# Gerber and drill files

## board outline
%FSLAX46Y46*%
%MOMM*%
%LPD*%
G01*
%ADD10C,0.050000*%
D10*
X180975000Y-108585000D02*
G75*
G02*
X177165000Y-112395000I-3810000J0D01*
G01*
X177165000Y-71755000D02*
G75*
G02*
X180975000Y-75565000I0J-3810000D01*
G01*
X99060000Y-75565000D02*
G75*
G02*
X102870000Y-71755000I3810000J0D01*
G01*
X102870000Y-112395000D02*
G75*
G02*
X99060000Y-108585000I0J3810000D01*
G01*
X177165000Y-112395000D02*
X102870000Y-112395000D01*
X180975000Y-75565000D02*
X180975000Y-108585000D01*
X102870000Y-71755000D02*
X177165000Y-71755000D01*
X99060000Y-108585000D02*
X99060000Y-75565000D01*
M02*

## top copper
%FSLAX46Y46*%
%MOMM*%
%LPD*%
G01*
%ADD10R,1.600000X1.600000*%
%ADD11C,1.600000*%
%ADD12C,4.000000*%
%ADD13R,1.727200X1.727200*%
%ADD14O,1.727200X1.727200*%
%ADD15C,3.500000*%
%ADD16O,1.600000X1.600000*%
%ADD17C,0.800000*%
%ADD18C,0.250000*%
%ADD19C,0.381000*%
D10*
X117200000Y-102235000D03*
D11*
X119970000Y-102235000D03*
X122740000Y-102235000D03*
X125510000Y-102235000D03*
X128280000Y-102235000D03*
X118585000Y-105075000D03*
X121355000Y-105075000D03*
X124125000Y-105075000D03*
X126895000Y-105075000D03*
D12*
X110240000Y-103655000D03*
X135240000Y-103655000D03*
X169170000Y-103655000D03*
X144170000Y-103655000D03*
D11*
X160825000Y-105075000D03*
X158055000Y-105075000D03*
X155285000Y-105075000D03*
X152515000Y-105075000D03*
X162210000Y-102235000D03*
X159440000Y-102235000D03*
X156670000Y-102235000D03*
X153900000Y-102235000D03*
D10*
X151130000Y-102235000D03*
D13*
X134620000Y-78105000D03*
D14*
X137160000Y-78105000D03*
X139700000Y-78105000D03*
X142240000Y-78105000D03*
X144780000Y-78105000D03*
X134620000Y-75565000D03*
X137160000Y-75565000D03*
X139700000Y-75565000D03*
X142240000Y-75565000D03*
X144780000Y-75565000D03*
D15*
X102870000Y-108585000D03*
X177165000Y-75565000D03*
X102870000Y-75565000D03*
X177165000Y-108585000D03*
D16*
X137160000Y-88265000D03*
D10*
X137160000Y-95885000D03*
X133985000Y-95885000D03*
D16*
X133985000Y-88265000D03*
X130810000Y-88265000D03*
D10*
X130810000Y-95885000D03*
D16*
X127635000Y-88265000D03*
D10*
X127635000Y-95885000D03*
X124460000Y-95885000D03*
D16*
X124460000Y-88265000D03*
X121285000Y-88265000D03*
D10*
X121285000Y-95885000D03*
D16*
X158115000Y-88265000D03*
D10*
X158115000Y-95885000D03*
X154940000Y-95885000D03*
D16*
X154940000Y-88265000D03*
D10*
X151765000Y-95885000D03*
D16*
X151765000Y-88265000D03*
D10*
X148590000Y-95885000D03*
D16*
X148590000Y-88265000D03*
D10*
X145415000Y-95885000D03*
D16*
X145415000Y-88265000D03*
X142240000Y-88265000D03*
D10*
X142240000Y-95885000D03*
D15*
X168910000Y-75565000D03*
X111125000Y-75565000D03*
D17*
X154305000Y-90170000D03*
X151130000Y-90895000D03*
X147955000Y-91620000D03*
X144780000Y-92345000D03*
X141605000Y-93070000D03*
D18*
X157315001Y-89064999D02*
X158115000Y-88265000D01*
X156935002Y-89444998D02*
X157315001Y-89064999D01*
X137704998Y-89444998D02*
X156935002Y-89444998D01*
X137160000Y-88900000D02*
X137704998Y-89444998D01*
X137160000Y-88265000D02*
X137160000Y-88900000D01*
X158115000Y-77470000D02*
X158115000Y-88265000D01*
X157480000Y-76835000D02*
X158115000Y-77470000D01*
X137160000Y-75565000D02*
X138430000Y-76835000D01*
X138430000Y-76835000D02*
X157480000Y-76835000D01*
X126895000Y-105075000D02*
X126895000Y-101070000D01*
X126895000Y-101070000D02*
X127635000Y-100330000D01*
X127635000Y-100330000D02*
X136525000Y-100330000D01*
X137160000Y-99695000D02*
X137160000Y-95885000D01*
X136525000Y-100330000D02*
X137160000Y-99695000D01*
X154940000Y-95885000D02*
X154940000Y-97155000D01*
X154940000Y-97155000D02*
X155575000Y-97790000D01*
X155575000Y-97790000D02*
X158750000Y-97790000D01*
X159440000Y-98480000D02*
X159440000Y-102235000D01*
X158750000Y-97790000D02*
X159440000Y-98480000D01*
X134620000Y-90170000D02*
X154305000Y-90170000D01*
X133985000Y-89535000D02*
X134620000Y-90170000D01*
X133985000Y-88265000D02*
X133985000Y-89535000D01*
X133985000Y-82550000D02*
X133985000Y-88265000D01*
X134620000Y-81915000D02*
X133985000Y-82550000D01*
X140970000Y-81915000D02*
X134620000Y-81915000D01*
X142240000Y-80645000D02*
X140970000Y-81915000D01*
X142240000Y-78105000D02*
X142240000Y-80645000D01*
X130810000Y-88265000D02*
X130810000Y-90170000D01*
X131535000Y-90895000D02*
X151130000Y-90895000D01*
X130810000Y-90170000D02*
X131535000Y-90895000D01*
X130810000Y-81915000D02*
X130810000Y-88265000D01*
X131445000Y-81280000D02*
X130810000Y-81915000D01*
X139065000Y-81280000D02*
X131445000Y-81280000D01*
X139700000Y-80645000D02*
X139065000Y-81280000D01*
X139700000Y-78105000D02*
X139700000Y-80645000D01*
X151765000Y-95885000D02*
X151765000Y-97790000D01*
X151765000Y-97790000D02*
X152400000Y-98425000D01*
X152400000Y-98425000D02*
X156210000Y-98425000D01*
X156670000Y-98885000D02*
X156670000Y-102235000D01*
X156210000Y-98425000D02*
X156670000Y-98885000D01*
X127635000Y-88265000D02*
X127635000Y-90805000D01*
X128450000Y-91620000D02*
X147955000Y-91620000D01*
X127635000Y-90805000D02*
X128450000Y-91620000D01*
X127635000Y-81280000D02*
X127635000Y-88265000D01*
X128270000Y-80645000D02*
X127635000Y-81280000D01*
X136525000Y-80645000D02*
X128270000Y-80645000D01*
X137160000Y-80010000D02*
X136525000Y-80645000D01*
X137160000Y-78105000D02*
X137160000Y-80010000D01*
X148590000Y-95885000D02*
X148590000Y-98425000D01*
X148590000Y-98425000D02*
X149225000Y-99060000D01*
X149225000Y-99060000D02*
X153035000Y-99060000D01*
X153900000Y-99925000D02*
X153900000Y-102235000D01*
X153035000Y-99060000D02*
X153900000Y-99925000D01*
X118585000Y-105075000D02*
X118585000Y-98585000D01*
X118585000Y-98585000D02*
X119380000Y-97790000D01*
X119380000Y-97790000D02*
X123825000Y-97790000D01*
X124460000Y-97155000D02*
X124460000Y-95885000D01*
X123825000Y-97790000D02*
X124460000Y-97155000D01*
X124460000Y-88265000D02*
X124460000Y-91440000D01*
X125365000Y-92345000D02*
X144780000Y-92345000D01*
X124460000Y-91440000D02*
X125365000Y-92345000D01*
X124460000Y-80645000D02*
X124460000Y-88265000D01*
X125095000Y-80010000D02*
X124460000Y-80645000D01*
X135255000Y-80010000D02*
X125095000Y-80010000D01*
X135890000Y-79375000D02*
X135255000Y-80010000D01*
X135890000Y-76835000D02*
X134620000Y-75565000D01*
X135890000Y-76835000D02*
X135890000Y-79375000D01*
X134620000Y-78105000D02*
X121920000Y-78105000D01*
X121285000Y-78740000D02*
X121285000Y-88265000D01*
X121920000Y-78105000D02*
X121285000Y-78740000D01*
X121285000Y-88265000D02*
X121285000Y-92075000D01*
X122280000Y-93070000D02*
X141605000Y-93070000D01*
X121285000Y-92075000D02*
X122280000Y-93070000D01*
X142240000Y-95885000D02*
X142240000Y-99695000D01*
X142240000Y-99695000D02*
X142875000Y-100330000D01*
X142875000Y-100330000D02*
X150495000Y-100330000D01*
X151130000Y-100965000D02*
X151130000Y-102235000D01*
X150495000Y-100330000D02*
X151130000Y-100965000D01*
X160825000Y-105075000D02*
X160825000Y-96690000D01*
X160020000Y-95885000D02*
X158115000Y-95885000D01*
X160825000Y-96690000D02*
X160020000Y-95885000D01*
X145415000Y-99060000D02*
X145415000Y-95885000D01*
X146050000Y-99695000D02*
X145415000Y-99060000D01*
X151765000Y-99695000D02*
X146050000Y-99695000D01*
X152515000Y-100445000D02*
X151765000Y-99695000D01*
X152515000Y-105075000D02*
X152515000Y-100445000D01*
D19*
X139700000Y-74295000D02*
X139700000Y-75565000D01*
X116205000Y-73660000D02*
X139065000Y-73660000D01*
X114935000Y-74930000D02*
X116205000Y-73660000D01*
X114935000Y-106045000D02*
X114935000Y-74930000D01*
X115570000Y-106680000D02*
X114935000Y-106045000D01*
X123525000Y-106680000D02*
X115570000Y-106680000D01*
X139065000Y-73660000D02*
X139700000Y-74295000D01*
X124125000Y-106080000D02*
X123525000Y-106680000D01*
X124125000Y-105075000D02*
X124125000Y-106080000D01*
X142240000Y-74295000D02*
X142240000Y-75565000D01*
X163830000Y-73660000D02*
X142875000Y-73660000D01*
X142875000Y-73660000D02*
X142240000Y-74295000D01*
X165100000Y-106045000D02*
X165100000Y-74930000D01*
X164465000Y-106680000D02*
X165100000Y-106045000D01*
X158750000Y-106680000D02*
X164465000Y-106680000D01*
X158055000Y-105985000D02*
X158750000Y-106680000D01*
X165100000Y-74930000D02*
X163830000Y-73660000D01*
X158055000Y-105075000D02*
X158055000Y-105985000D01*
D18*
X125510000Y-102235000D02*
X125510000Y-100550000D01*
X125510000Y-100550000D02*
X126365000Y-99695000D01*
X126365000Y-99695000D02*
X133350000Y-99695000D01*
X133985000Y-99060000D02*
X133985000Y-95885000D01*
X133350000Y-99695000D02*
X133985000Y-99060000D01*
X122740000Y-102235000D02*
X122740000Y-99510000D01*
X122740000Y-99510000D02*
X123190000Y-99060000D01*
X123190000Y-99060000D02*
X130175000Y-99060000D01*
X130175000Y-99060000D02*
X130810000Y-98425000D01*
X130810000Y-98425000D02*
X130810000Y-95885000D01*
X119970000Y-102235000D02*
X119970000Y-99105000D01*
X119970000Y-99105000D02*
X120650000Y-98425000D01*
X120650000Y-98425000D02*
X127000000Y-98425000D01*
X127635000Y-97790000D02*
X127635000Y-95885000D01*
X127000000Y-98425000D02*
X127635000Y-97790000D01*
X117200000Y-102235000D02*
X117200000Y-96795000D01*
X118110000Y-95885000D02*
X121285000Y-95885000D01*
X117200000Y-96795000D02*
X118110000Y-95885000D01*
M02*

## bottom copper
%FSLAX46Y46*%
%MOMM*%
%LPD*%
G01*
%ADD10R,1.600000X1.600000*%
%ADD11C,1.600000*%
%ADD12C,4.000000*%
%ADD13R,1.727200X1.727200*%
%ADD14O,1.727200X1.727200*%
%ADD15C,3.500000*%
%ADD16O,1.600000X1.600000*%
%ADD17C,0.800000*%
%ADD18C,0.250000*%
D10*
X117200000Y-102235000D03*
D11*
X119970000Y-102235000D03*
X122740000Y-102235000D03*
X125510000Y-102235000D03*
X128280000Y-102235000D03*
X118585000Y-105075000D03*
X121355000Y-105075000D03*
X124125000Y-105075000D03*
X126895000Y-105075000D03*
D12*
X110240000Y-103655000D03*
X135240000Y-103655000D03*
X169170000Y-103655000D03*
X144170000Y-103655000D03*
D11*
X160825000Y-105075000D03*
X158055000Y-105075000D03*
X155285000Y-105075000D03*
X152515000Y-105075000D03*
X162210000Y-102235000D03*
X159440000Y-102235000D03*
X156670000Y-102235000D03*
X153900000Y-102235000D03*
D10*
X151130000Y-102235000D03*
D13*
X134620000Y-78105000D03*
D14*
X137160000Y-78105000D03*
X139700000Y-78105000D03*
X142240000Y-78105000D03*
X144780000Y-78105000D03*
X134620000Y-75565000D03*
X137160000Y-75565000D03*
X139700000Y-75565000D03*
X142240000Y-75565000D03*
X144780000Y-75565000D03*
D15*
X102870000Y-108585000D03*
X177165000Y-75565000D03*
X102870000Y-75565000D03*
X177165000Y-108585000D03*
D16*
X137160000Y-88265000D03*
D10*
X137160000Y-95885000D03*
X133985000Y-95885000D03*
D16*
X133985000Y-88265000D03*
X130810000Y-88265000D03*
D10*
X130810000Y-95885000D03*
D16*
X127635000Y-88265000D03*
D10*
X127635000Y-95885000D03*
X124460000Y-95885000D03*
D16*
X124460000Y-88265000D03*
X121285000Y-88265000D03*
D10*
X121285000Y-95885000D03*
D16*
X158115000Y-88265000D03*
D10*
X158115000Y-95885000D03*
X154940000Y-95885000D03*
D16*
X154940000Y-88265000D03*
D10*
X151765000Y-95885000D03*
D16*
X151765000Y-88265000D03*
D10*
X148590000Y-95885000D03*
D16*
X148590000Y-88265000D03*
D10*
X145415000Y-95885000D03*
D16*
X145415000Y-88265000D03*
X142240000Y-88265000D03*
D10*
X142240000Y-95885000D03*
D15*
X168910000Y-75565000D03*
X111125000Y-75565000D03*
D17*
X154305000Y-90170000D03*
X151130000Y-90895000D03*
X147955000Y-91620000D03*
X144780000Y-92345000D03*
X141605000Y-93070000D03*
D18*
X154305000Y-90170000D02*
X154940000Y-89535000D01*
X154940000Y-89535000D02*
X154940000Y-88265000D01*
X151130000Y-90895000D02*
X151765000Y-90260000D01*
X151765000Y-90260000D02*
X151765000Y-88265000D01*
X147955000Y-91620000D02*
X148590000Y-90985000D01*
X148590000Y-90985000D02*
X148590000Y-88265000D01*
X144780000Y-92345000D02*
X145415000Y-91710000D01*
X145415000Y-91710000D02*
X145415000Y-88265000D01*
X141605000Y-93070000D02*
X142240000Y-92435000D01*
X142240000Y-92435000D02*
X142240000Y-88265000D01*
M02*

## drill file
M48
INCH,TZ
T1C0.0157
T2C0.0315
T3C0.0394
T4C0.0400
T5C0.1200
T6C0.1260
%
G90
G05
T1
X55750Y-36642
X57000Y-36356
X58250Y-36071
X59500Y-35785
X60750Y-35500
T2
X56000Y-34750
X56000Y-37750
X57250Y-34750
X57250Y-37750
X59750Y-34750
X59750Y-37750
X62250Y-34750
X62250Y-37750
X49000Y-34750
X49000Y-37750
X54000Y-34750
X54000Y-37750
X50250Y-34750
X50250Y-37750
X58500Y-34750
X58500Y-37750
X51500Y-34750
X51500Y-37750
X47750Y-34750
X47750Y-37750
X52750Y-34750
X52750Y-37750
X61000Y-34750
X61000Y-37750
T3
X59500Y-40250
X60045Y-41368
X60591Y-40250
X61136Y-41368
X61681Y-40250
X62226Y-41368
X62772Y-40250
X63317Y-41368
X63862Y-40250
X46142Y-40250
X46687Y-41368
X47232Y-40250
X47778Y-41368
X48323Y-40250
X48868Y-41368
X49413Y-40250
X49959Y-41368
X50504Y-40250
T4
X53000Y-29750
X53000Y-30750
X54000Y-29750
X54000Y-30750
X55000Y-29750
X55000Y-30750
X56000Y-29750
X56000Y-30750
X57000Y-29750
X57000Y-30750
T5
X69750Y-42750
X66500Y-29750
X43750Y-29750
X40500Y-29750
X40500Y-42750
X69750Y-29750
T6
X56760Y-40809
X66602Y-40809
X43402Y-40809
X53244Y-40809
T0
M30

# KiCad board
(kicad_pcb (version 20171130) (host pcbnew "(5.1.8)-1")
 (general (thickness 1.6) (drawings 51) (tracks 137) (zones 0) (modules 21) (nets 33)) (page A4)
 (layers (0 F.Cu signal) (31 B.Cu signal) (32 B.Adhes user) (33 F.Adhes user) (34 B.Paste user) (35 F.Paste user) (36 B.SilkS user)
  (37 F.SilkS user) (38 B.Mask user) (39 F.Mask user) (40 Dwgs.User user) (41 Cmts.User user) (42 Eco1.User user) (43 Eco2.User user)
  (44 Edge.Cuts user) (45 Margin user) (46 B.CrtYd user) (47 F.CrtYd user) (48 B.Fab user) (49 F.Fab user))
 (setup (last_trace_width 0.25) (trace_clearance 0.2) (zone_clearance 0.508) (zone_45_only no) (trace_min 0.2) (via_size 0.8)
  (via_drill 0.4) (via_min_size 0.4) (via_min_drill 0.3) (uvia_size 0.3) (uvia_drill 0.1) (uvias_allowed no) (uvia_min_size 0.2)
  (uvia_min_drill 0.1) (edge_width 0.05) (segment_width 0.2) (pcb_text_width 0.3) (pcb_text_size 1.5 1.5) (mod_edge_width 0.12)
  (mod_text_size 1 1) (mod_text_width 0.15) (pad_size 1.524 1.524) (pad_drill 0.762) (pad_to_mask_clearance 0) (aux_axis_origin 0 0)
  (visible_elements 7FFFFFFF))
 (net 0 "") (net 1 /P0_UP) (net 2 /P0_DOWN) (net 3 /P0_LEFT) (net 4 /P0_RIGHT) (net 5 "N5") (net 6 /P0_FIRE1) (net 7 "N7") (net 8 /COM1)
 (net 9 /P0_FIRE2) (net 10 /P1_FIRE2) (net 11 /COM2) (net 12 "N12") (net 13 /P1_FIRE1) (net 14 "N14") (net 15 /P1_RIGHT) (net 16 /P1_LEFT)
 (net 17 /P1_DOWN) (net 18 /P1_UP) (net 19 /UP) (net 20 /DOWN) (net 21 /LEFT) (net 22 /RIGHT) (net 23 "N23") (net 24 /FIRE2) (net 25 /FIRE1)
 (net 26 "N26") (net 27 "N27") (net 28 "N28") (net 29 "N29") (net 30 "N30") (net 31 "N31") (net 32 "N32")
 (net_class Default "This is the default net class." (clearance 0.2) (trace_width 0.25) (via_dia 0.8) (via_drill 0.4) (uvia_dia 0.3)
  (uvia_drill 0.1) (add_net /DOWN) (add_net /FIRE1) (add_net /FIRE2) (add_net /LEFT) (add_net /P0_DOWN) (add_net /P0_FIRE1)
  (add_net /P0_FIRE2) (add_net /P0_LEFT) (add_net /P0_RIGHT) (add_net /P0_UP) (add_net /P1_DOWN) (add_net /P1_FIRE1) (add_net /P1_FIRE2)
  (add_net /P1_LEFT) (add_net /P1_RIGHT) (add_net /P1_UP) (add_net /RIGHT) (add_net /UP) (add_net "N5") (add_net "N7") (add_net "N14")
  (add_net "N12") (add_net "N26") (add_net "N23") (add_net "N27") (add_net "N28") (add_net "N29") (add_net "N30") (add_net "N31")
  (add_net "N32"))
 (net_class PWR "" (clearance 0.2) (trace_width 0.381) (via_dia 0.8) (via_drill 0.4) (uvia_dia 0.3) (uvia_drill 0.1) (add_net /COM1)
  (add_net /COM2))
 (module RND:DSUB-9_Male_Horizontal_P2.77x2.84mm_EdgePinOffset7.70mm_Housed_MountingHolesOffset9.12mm (layer F.Cu) (at 117.2 102.235)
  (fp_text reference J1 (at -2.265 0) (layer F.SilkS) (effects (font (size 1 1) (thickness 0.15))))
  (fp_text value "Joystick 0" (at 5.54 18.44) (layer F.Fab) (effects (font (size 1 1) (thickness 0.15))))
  (pad 1 thru_hole rect (at 0 0) (size 1.6 1.6) (drill 1) (layers *.Cu *.Mask) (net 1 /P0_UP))
  (pad 2 thru_hole circle (at 2.77 0) (size 1.6 1.6) (drill 1) (layers *.Cu *.Mask) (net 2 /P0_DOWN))
  (pad 3 thru_hole circle (at 5.54 0) (size 1.6 1.6) (drill 1) (layers *.Cu *.Mask) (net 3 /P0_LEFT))
  (pad 4 thru_hole circle (at 8.31 0) (size 1.6 1.6) (drill 1) (layers *.Cu *.Mask) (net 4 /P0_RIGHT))
  (pad 5 thru_hole circle (at 11.08 0) (size 1.6 1.6) (drill 1) (layers *.Cu *.Mask) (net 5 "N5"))
  (pad 6 thru_hole circle (at 1.385 2.84) (size 1.6 1.6) (drill 1) (layers *.Cu *.Mask) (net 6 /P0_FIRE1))
  (pad 7 thru_hole circle (at 4.155 2.84) (size 1.6 1.6) (drill 1) (layers *.Cu *.Mask) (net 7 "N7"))
  (pad 8 thru_hole circle (at 6.925 2.84) (size 1.6 1.6) (drill 1) (layers *.Cu *.Mask) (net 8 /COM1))
  (pad 9 thru_hole circle (at 9.695 2.84) (size 1.6 1.6) (drill 1) (layers *.Cu *.Mask) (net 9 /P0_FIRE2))
  (pad 0 thru_hole circle (at -6.96 1.42) (size 4 4) (drill 3.2) (layers *.Cu *.Mask))
  (pad 0 thru_hole circle (at 18.04 1.42) (size 4 4) (drill 3.2) (layers *.Cu *.Mask)))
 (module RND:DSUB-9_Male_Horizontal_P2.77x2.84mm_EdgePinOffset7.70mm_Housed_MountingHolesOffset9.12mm (layer F.Cu) (at 151.13 102.235)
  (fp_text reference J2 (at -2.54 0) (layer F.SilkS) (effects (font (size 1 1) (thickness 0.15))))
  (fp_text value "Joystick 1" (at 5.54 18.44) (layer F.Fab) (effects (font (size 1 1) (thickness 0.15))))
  (pad 0 thru_hole circle (at 18.04 1.42) (size 4 4) (drill 3.2) (layers *.Cu *.Mask))
  (pad 0 thru_hole circle (at -6.96 1.42) (size 4 4) (drill 3.2) (layers *.Cu *.Mask))
  (pad 9 thru_hole circle (at 9.695 2.84) (size 1.6 1.6) (drill 1) (layers *.Cu *.Mask) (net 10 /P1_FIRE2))
  (pad 8 thru_hole circle (at 6.925 2.84) (size 1.6 1.6) (drill 1) (layers *.Cu *.Mask) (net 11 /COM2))
  (pad 7 thru_hole circle (at 4.155 2.84) (size 1.6 1.6) (drill 1) (layers *.Cu *.Mask) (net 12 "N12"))
  (pad 6 thru_hole circle (at 1.385 2.84) (size 1.6 1.6) (drill 1) (layers *.Cu *.Mask) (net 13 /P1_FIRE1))
  (pad 5 thru_hole circle (at 11.08 0) (size 1.6 1.6) (drill 1) (layers *.Cu *.Mask) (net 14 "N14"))
  (pad 4 thru_hole circle (at 8.31 0) (size 1.6 1.6) (drill 1) (layers *.Cu *.Mask) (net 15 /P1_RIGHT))
  (pad 3 thru_hole circle (at 5.54 0) (size 1.6 1.6) (drill 1) (layers *.Cu *.Mask) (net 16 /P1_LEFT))
  (pad 2 thru_hole circle (at 2.77 0) (size 1.6 1.6) (drill 1) (layers *.Cu *.Mask) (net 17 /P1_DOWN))
  (pad 1 thru_hole rect (at 0 0) (size 1.6 1.6) (drill 1) (layers *.Cu *.Mask) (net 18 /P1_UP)))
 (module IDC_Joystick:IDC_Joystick (layer F.Cu) (at 134.62 78.105 90)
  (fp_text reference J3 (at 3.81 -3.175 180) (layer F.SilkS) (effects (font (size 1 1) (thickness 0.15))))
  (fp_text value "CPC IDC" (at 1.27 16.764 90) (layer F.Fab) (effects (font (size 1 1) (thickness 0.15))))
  (pad 1 thru_hole rect (at 0 0 90) (size 1.7272 1.7272) (drill 1.016) (layers *.Cu *.Mask) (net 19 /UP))
  (pad 2 thru_hole oval (at 0 2.54 90) (size 1.7272 1.7272) (drill 1.016) (layers *.Cu *.Mask) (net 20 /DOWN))
  (pad 3 thru_hole oval (at 0 5.08 90) (size 1.7272 1.7272) (drill 1.016) (layers *.Cu *.Mask) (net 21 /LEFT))
  (pad 4 thru_hole oval (at 0 7.62 90) (size 1.7272 1.7272) (drill 1.016) (layers *.Cu *.Mask) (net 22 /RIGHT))
  (pad 5 thru_hole oval (at 0 10.16 90) (size 1.7272 1.7272) (drill 1.016) (layers *.Cu *.Mask) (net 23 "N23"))
  (pad 6 thru_hole oval (at 2.54 0 90) (size 1.7272 1.7272) (drill 1.016) (layers *.Cu *.Mask) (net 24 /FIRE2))
  (pad 7 thru_hole oval (at 2.54 2.54 90) (size 1.7272 1.7272) (drill 1.016) (layers *.Cu *.Mask) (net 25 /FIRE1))
  (pad 8 thru_hole oval (at 2.54 5.08 90) (size 1.7272 1.7272) (drill 1.016) (layers *.Cu *.Mask) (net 8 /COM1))
  (pad 9 thru_hole oval (at 2.54 7.62 90) (size 1.7272 1.7272) (drill 1.016) (layers *.Cu *.Mask) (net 11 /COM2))
  (pad 10 thru_hole oval (at 2.54 10.16 90) (size 1.7272 1.7272) (drill 1.016) (layers *.Cu *.Mask) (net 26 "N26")))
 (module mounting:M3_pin (layer F.Cu) (at 102.87 108.585)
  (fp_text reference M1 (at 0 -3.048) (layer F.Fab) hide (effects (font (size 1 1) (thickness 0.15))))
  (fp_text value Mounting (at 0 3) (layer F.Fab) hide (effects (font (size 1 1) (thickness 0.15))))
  (pad 1 thru_hole circle (at 0 0) (size 3.5 3.5) (drill 3.048) (layers *.Cu *.Mask) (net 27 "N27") (solder_mask_margin 0.8)))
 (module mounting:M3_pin (layer F.Cu) (at 177.165 75.565)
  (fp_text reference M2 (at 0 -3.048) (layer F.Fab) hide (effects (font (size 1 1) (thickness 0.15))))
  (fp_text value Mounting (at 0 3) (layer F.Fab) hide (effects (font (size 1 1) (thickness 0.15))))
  (pad 1 thru_hole circle (at 0 0) (size 3.5 3.5) (drill 3.048) (layers *.Cu *.Mask) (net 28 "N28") (solder_mask_margin 0.8)))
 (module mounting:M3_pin (layer F.Cu) (at 102.87 75.565)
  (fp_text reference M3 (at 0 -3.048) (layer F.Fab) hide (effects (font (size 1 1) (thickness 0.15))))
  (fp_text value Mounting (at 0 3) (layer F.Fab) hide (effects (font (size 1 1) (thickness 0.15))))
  (pad 1 thru_hole circle (at 0 0) (size 3.5 3.5) (drill 3.048) (layers *.Cu *.Mask) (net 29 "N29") (solder_mask_margin 0.8)))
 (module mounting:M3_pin (layer F.Cu) (at 177.165 108.585)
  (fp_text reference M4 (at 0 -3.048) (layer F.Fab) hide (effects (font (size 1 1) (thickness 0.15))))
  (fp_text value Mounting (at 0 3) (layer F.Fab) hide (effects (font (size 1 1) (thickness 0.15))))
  (pad 1 thru_hole circle (at 0 0) (size 3.5 3.5) (drill 3.048) (layers *.Cu *.Mask) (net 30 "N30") (solder_mask_margin 0.8)))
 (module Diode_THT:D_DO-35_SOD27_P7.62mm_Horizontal (layer F.Cu) (at 137.16 95.885 90)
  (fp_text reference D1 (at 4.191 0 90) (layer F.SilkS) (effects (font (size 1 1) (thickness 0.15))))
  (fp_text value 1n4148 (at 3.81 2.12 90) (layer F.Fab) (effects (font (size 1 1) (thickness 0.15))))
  (pad 2 thru_hole oval (at 7.62 0 90) (size 1.6 1.6) (drill 0.8) (layers *.Cu *.Mask) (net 25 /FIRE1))
  (pad 1 thru_hole rect (at 0 0 90) (size 1.6 1.6) (drill 0.8) (layers *.Cu *.Mask) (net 9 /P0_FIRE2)))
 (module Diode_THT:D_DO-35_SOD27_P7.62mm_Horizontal (layer F.Cu) (at 133.985 95.885 90)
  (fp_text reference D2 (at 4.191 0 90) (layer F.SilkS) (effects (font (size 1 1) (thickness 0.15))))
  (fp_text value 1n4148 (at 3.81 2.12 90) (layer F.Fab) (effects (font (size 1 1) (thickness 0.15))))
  (pad 1 thru_hole rect (at 0 0 90) (size 1.6 1.6) (drill 0.8) (layers *.Cu *.Mask) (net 4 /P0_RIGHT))
  (pad 2 thru_hole oval (at 7.62 0 90) (size 1.6 1.6) (drill 0.8) (layers *.Cu *.Mask) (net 22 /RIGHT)))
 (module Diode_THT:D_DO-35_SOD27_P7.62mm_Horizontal (layer F.Cu) (at 130.81 95.885 90)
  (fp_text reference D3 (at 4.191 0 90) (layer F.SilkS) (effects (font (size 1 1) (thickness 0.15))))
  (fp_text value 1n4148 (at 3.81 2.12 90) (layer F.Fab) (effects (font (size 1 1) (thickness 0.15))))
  (pad 2 thru_hole oval (at 7.62 0 90) (size 1.6 1.6) (drill 0.8) (layers *.Cu *.Mask) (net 21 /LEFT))
  (pad 1 thru_hole rect (at 0 0 90) (size 1.6 1.6) (drill 0.8) (layers *.Cu *.Mask) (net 3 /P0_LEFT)))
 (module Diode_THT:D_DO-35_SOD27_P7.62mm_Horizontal (layer F.Cu) (at 127.635 95.885 90)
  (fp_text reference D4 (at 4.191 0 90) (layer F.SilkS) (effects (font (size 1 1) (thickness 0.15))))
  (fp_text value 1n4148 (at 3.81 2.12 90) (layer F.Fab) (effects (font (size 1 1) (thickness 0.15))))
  (pad 2 thru_hole oval (at 7.62 0 90) (size 1.6 1.6) (drill 0.8) (layers *.Cu *.Mask) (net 20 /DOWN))
  (pad 1 thru_hole rect (at 0 0 90) (size 1.6 1.6) (drill 0.8) (layers *.Cu *.Mask) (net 2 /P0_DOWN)))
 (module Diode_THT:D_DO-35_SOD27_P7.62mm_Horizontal (layer F.Cu) (at 124.46 95.885 90)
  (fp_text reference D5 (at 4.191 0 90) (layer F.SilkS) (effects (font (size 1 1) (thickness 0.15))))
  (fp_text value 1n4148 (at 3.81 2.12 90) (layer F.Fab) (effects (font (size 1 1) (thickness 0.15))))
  (pad 1 thru_hole rect (at 0 0 90) (size 1.6 1.6) (drill 0.8) (layers *.Cu *.Mask) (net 6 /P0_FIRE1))
  (pad 2 thru_hole oval (at 7.62 0 90) (size 1.6 1.6) (drill 0.8) (layers *.Cu *.Mask) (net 24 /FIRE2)))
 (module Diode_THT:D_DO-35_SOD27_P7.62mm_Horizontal (layer F.Cu) (at 121.285 95.885 90)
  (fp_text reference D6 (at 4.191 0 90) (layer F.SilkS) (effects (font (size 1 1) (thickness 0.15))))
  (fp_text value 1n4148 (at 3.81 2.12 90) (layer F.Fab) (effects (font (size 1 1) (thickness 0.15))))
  (pad 2 thru_hole oval (at 7.62 0 90) (size 1.6 1.6) (drill 0.8) (layers *.Cu *.Mask) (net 19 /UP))
  (pad 1 thru_hole rect (at 0 0 90) (size 1.6 1.6) (drill 0.8) (layers *.Cu *.Mask) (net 1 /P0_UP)))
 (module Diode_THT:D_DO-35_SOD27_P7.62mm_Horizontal (layer F.Cu) (at 158.115 95.885 90)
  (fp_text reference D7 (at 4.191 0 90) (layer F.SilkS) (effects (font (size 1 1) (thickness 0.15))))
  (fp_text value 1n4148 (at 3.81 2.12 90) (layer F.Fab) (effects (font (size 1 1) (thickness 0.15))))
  (pad 2 thru_hole oval (at 7.62 0 90) (size 1.6 1.6) (drill 0.8) (layers *.Cu *.Mask) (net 25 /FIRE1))
  (pad 1 thru_hole rect (at 0 0 90) (size 1.6 1.6) (drill 0.8) (layers *.Cu *.Mask) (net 10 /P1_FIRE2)))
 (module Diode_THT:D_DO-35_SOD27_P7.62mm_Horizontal (layer F.Cu) (at 154.94 95.885 90)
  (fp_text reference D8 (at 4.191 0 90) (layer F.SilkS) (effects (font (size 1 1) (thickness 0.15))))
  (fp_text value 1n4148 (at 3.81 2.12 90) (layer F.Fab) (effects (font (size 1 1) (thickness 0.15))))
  (pad 1 thru_hole rect (at 0 0 90) (size 1.6 1.6) (drill 0.8) (layers *.Cu *.Mask) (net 15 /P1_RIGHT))
  (pad 2 thru_hole oval (at 7.62 0 90) (size 1.6 1.6) (drill 0.8) (layers *.Cu *.Mask) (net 22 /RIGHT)))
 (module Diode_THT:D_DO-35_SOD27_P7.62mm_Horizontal (layer F.Cu) (at 151.765 95.885 90)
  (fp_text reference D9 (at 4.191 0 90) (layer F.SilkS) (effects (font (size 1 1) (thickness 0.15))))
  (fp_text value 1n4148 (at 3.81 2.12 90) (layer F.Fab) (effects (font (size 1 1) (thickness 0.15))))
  (pad 1 thru_hole rect (at 0 0 90) (size 1.6 1.6) (drill 0.8) (layers *.Cu *.Mask) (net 16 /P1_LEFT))
  (pad 2 thru_hole oval (at 7.62 0 90) (size 1.6 1.6) (drill 0.8) (layers *.Cu *.Mask) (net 21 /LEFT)))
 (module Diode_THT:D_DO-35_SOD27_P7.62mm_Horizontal (layer F.Cu) (at 148.59 95.885 90)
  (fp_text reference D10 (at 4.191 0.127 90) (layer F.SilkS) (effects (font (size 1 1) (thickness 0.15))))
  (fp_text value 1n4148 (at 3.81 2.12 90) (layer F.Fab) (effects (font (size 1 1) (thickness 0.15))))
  (pad 1 thru_hole rect (at 0 0 90) (size 1.6 1.6) (drill 0.8) (layers *.Cu *.Mask) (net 17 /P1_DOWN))
  (pad 2 thru_hole oval (at 7.62 0 90) (size 1.6 1.6) (drill 0.8) (layers *.Cu *.Mask) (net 20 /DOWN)))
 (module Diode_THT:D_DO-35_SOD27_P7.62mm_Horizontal (layer F.Cu) (at 145.415 95.885 90)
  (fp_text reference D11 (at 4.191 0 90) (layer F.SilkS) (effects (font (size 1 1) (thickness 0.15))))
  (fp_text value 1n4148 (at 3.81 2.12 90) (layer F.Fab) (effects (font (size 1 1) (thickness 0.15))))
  (pad 1 thru_hole rect (at 0 0 90) (size 1.6 1.6) (drill 0.8) (layers *.Cu *.Mask) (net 13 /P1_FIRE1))
  (pad 2 thru_hole oval (at 7.62 0 90) (size 1.6 1.6) (drill 0.8) (layers *.Cu *.Mask) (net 24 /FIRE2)))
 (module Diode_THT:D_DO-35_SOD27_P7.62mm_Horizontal (layer F.Cu) (at 142.24 95.885 90)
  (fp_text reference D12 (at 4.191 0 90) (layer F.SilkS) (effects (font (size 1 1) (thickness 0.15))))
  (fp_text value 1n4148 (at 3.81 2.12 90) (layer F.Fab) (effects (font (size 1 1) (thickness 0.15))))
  (pad 2 thru_hole oval (at 7.62 0 90) (size 1.6 1.6) (drill 0.8) (layers *.Cu *.Mask) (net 19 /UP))
  (pad 1 thru_hole rect (at 0 0 90) (size 1.6 1.6) (drill 0.8) (layers *.Cu *.Mask) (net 18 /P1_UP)))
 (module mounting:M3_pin (layer F.Cu) (at 168.91 75.565)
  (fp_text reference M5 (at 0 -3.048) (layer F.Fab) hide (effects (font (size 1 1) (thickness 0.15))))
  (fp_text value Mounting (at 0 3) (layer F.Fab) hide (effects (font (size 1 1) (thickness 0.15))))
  (pad 1 thru_hole circle (at 0 0) (size 3.5 3.5) (drill 3.048) (layers *.Cu *.Mask) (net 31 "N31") (solder_mask_margin 0.8)))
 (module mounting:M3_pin (layer F.Cu) (at 111.125 75.565)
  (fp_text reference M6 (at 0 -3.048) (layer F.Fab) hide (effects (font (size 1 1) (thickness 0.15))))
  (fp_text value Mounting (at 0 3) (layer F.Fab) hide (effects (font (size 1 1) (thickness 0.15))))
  (pad 1 thru_hole circle (at 0 0) (size 3.5 3.5) (drill 3.048) (layers *.Cu *.Mask) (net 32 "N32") (solder_mask_margin 0.8)))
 (gr_arc (start 177.165 108.585) (end 177.165 112.395) (angle -90) (layer Edge.Cuts) (width 0.05))
 (gr_arc (start 177.165 75.565) (end 180.975 75.565) (angle -90) (layer Edge.Cuts) (width 0.05))
 (gr_arc (start 102.87 75.565) (end 102.87 71.755) (angle -90) (layer Edge.Cuts) (width 0.05))
 (gr_arc (start 102.87 108.585) (end 99.06 108.585) (angle -90) (layer Edge.Cuts) (width 0.05))
 (gr_line (start 177.165 112.395) (end 102.87 112.395) (layer Edge.Cuts) (width 0.05))
 (gr_line (start 180.975 75.565) (end 180.975 108.585) (layer Edge.Cuts) (width 0.05))
 (gr_line (start 102.87 71.755) (end 177.165 71.755) (layer Edge.Cuts) (width 0.05))
 (gr_line (start 99.06 108.585) (end 99.06 75.565) (layer Edge.Cuts) (width 0.05))
 (segment (start 157.315001 89.064999) (end 158.115 88.265) (width 0.25) (layer F.Cu) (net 25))
 (segment (start 156.935002 89.444998) (end 157.315001 89.064999) (width 0.25) (layer F.Cu) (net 25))
 (segment (start 137.704998 89.444998) (end 156.935002 89.444998) (width 0.25) (layer F.Cu) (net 25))
 (segment (start 137.16 88.9) (end 137.704998 89.444998) (width 0.25) (layer F.Cu) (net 25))
 (segment (start 137.16 88.265) (end 137.16 88.9) (width 0.25) (layer F.Cu) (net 25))
 (segment (start 158.115 77.47) (end 158.115 88.265) (width 0.25) (layer F.Cu) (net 25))
 (segment (start 157.48 76.835) (end 158.115 77.47) (width 0.25) (layer F.Cu) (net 25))
 (segment (start 137.16 75.565) (end 138.43 76.835) (width 0.25) (layer F.Cu) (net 25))
 (segment (start 138.43 76.835) (end 157.48 76.835) (width 0.25) (layer F.Cu) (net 25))
 (segment (start 126.895 105.075) (end 126.895 101.07) (width 0.25) (layer F.Cu) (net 9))
 (segment (start 126.895 101.07) (end 127.635 100.33) (width 0.25) (layer F.Cu) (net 9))
 (segment (start 127.635 100.33) (end 136.525 100.33) (width 0.25) (layer F.Cu) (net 9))
 (segment (start 137.16 99.695) (end 137.16 95.885) (width 0.25) (layer F.Cu) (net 9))
 (segment (start 136.525 100.33) (end 137.16 99.695) (width 0.25) (layer F.Cu) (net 9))
 (segment (start 154.94 95.885) (end 154.94 97.155) (width 0.25) (layer F.Cu) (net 15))
 (segment (start 154.94 97.155) (end 155.575 97.79) (width 0.25) (layer F.Cu) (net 15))
 (segment (start 155.575 97.79) (end 158.75 97.79) (width 0.25) (layer F.Cu) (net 15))
 (segment (start 159.44 98.48) (end 159.44 102.235) (width 0.25) (layer F.Cu) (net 15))
 (segment (start 158.75 97.79) (end 159.44 98.48) (width 0.25) (layer F.Cu) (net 15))
 (via (at 154.305 90.17) (size 0.8) (drill 0.4) (layers F.Cu B.Cu) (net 22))
 (segment (start 154.305 90.17) (end 154.94 89.535) (width 0.25) (layer B.Cu) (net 22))
 (segment (start 154.94 89.535) (end 154.94 88.265) (width 0.25) (layer B.Cu) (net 22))
 (segment (start 134.62 90.17) (end 154.305 90.17) (width 0.25) (layer F.Cu) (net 22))
 (segment (start 133.985 89.535) (end 134.62 90.17) (width 0.25) (layer F.Cu) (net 22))
 (segment (start 133.985 88.265) (end 133.985 89.535) (width 0.25) (layer F.Cu) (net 22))
 (segment (start 133.985 82.55) (end 133.985 88.265) (width 0.25) (layer F.Cu) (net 22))
 (segment (start 134.62 81.915) (end 133.985 82.55) (width 0.25) (layer F.Cu) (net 22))
 (segment (start 140.97 81.915) (end 134.62 81.915) (width 0.25) (layer F.Cu) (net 22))
 (segment (start 142.24 80.645) (end 140.97 81.915) (width 0.25) (layer F.Cu) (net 22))
 (segment (start 142.24 78.105) (end 142.24 80.645) (width 0.25) (layer F.Cu) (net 22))
 (segment (start 130.81 88.265) (end 130.81 90.17) (width 0.25) (layer F.Cu) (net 21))
 (via (at 151.13 90.895) (size 0.8) (drill 0.4) (layers F.Cu B.Cu) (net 21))
 (segment (start 131.535 90.895) (end 151.13 90.895) (width 0.25) (layer F.Cu) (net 21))
 (segment (start 130.81 90.17) (end 131.535 90.895) (width 0.25) (layer F.Cu) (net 21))
 (segment (start 151.13 90.895) (end 151.765 90.26) (width 0.25) (layer B.Cu) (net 21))
 (segment (start 151.765 90.26) (end 151.765 88.265) (width 0.25) (layer B.Cu) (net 21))
 (segment (start 130.81 81.915) (end 130.81 88.265) (width 0.25) (layer F.Cu) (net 21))
 (segment (start 131.445 81.28) (end 130.81 81.915) (width 0.25) (layer F.Cu) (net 21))
 (segment (start 139.065 81.28) (end 131.445 81.28) (width 0.25) (layer F.Cu) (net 21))
 (segment (start 139.7 80.645) (end 139.065 81.28) (width 0.25) (layer F.Cu) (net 21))
 (segment (start 139.7 78.105) (end 139.7 80.645) (width 0.25) (layer F.Cu) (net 21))
 (segment (start 151.765 95.885) (end 151.765 97.79) (width 0.25) (layer F.Cu) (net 16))
 (segment (start 151.765 97.79) (end 152.4 98.425) (width 0.25) (layer F.Cu) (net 16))
 (segment (start 152.4 98.425) (end 156.21 98.425) (width 0.25) (layer F.Cu) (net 16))
 (segment (start 156.67 98.885) (end 156.67 102.235) (width 0.25) (layer F.Cu) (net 16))
 (segment (start 156.21 98.425) (end 156.67 98.885) (width 0.25) (layer F.Cu) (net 16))
 (segment (start 127.635 88.265) (end 127.635 90.805) (width 0.25) (layer F.Cu) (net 20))
 (via (at 147.955 91.62) (size 0.8) (drill 0.4) (layers F.Cu B.Cu) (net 20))
 (segment (start 128.45 91.62) (end 147.955 91.62) (width 0.25) (layer F.Cu) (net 20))
 (segment (start 127.635 90.805) (end 128.45 91.62) (width 0.25) (layer F.Cu) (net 20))
 (segment (start 147.955 91.62) (end 148.59 90.985) (width 0.25) (layer B.Cu) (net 20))
 (segment (start 148.59 90.985) (end 148.59 88.265) (width 0.25) (layer B.Cu) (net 20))
 (segment (start 127.635 81.28) (end 127.635 88.265) (width 0.25) (layer F.Cu) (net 20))
 (segment (start 128.27 80.645) (end 127.635 81.28) (width 0.25) (layer F.Cu) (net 20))
 (segment (start 136.525 80.645) (end 128.27 80.645) (width 0.25) (layer F.Cu) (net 20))
 (segment (start 137.16 80.01) (end 136.525 80.645) (width 0.25) (layer F.Cu) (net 20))
 (segment (start 137.16 78.105) (end 137.16 80.01) (width 0.25) (layer F.Cu) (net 20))
 (segment (start 148.59 95.885) (end 148.59 98.425) (width 0.25) (layer F.Cu) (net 17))
 (segment (start 148.59 98.425) (end 149.225 99.06) (width 0.25) (layer F.Cu) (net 17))
 (segment (start 149.225 99.06) (end 153.035 99.06) (width 0.25) (layer F.Cu) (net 17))
 (segment (start 153.9 99.925) (end 153.9 102.235) (width 0.25) (layer F.Cu) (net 17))
 (segment (start 153.035 99.06) (end 153.9 99.925) (width 0.25) (layer F.Cu) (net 17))
 (segment (start 118.585 105.075) (end 118.585 98.585) (width 0.25) (layer F.Cu) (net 6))
 (segment (start 118.585 98.585) (end 119.38 97.79) (width 0.25) (layer F.Cu) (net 6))
 (segment (start 119.38 97.79) (end 123.825 97.79) (width 0.25) (layer F.Cu) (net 6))
 (segment (start 124.46 97.155) (end 124.46 95.885) (width 0.25) (layer F.Cu) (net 6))
 (segment (start 123.825 97.79) (end 124.46 97.155) (width 0.25) (layer F.Cu) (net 6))
 (segment (start 124.46 88.265) (end 124.46 91.44) (width 0.25) (layer F.Cu) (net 24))
 (via (at 144.78 92.345) (size 0.8) (drill 0.4) (layers F.Cu B.Cu) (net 24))
 (segment (start 125.365 92.345) (end 144.78 92.345) (width 0.25) (layer F.Cu) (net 24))
 (segment (start 124.46 91.44) (end 125.365 92.345) (width 0.25) (layer F.Cu) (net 24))
 (segment (start 144.78 92.345) (end 145.415 91.71) (width 0.25) (layer B.Cu) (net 24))
 (segment (start 145.415 91.71) (end 145.415 88.265) (width 0.25) (layer B.Cu) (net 24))
 (segment (start 124.46 80.645) (end 124.46 88.265) (width 0.25) (layer F.Cu) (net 24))
 (segment (start 125.095 80.01) (end 124.46 80.645) (width 0.25) (layer F.Cu) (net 24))
 (segment (start 135.255 80.01) (end 125.095 80.01) (width 0.25) (layer F.Cu) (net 24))
 (segment (start 135.89 79.375) (end 135.255 80.01) (width 0.25) (layer F.Cu) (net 24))
 (segment (start 135.89 76.835) (end 134.62 75.565) (width 0.25) (layer F.Cu) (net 24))
 (segment (start 135.89 76.835) (end 135.89 79.375) (width 0.25) (layer F.Cu) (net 24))
 (segment (start 134.62 78.105) (end 121.92 78.105) (width 0.25) (layer F.Cu) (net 19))
 (segment (start 121.285 78.74) (end 121.285 88.265) (width 0.25) (layer F.Cu) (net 19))
 (segment (start 121.92 78.105) (end 121.285 78.74) (width 0.25) (layer F.Cu) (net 19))
 (segment (start 121.285 88.265) (end 121.285 92.075) (width 0.25) (layer F.Cu) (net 19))
 (via (at 141.605 93.07) (size 0.8) (drill 0.4) (layers F.Cu B.Cu) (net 19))
 (segment (start 122.28 93.07) (end 141.605 93.07) (width 0.25) (layer F.Cu) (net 19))
 (segment (start 121.285 92.075) (end 122.28 93.07) (width 0.25) (layer F.Cu) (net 19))
 (segment (start 141.605 93.07) (end 142.24 92.435) (width 0.25) (layer B.Cu) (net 19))
 (segment (start 142.24 92.435) (end 142.24 88.265) (width 0.25) (layer B.Cu) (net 19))
 (segment (start 142.24 95.885) (end 142.24 99.695) (width 0.25) (layer F.Cu) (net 18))
 (segment (start 142.24 99.695) (end 142.875 100.33) (width 0.25) (layer F.Cu) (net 18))
 (segment (start 142.875 100.33) (end 150.495 100.33) (width 0.25) (layer F.Cu) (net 18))
 (segment (start 151.13 100.965) (end 151.13 102.235) (width 0.25) (layer F.Cu) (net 18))
 (segment (start 150.495 100.33) (end 151.13 100.965) (width 0.25) (layer F.Cu) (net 18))
 (segment (start 160.825 105.075) (end 160.825 96.69) (width 0.25) (layer F.Cu) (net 10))
 (segment (start 160.02 95.885) (end 158.115 95.885) (width 0.25) (layer F.Cu) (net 10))
 (segment (start 160.825 96.69) (end 160.02 95.885) (width 0.25) (layer F.Cu) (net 10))
 (segment (start 145.415 99.06) (end 145.415 95.885) (width 0.25) (layer F.Cu) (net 13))
 (segment (start 146.05 99.695) (end 145.415 99.06) (width 0.25) (layer F.Cu) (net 13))
 (segment (start 151.765 99.695) (end 146.05 99.695) (width 0.25) (layer F.Cu) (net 13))
 (segment (start 152.515 100.445) (end 151.765 99.695) (width 0.25) (layer F.Cu) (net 13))
 (segment (start 152.515 105.075) (end 152.515 100.445) (width 0.25) (layer F.Cu) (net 13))
 (segment (start 139.7 74.295) (end 139.7 75.565) (width 0.381) (layer F.Cu) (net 8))
 (segment (start 116.205 73.66) (end 139.065 73.66) (width 0.381) (layer F.Cu) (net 8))
 (segment (start 114.935 74.93) (end 116.205 73.66) (width 0.381) (layer F.Cu) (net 8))
 (segment (start 114.935 106.045) (end 114.935 74.93) (width 0.381) (layer F.Cu) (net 8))
 (segment (start 115.57 106.68) (end 114.935 106.045) (width 0.381) (layer F.Cu) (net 8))
 (segment (start 123.525 106.68) (end 115.57 106.68) (width 0.381) (layer F.Cu) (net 8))
 (segment (start 139.065 73.66) (end 139.7 74.295) (width 0.381) (layer F.Cu) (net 8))
 (segment (start 124.125 106.08) (end 123.525 106.68) (width 0.381) (layer F.Cu) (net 8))
 (segment (start 124.125 105.075) (end 124.125 106.08) (width 0.381) (layer F.Cu) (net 8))
 (segment (start 142.24 74.295) (end 142.24 75.565) (width 0.381) (layer F.Cu) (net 11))
 (segment (start 163.83 73.66) (end 142.875 73.66) (width 0.381) (layer F.Cu) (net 11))
 (segment (start 142.875 73.66) (end 142.24 74.295) (width 0.381) (layer F.Cu) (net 11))
 (segment (start 165.1 106.045) (end 165.1 74.93) (width 0.381) (layer F.Cu) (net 11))
 (segment (start 164.465 106.68) (end 165.1 106.045) (width 0.381) (layer F.Cu) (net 11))
 (segment (start 158.75 106.68) (end 164.465 106.68) (width 0.381) (layer F.Cu) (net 11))
 (segment (start 158.055 105.985) (end 158.75 106.68) (width 0.381) (layer F.Cu) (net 11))
 (segment (start 165.1 74.93) (end 163.83 73.66) (width 0.381) (layer F.Cu) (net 11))
 (segment (start 158.055 105.075) (end 158.055 105.985) (width 0.381) (layer F.Cu) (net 11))
 (segment (start 125.51 102.235) (end 125.51 100.55) (width 0.25) (layer F.Cu) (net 4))
 (segment (start 125.51 100.55) (end 126.365 99.695) (width 0.25) (layer F.Cu) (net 4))
 (segment (start 126.365 99.695) (end 133.35 99.695) (width 0.25) (layer F.Cu) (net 4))
 (segment (start 133.985 99.06) (end 133.985 95.885) (width 0.25) (layer F.Cu) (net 4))
 (segment (start 133.35 99.695) (end 133.985 99.06) (width 0.25) (layer F.Cu) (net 4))
 (segment (start 122.74 102.235) (end 122.74 99.51) (width 0.25) (layer F.Cu) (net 3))
 (segment (start 122.74 99.51) (end 123.19 99.06) (width 0.25) (layer F.Cu) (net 3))
 (segment (start 123.19 99.06) (end 130.175 99.06) (width 0.25) (layer F.Cu) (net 3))
 (segment (start 130.175 99.06) (end 130.81 98.425) (width 0.25) (layer F.Cu) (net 3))
 (segment (start 130.81 98.425) (end 130.81 95.885) (width 0.25) (layer F.Cu) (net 3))
 (segment (start 119.97 102.235) (end 119.97 99.105) (width 0.25) (layer F.Cu) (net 2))
 (segment (start 119.97 99.105) (end 120.65 98.425) (width 0.25) (layer F.Cu) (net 2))
 (segment (start 120.65 98.425) (end 127 98.425) (width 0.25) (layer F.Cu) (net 2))
 (segment (start 127.635 97.79) (end 127.635 95.885) (width 0.25) (layer F.Cu) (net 2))
 (segment (start 127 98.425) (end 127.635 97.79) (width 0.25) (layer F.Cu) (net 2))
 (segment (start 117.2 102.235) (end 117.2 96.795) (width 0.25) (layer F.Cu) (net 1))
 (segment (start 118.11 95.885) (end 121.285 95.885) (width 0.25) (layer F.Cu) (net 1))
 (segment (start 117.2 96.795) (end 118.11 95.885) (width 0.25) (layer F.Cu) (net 1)))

